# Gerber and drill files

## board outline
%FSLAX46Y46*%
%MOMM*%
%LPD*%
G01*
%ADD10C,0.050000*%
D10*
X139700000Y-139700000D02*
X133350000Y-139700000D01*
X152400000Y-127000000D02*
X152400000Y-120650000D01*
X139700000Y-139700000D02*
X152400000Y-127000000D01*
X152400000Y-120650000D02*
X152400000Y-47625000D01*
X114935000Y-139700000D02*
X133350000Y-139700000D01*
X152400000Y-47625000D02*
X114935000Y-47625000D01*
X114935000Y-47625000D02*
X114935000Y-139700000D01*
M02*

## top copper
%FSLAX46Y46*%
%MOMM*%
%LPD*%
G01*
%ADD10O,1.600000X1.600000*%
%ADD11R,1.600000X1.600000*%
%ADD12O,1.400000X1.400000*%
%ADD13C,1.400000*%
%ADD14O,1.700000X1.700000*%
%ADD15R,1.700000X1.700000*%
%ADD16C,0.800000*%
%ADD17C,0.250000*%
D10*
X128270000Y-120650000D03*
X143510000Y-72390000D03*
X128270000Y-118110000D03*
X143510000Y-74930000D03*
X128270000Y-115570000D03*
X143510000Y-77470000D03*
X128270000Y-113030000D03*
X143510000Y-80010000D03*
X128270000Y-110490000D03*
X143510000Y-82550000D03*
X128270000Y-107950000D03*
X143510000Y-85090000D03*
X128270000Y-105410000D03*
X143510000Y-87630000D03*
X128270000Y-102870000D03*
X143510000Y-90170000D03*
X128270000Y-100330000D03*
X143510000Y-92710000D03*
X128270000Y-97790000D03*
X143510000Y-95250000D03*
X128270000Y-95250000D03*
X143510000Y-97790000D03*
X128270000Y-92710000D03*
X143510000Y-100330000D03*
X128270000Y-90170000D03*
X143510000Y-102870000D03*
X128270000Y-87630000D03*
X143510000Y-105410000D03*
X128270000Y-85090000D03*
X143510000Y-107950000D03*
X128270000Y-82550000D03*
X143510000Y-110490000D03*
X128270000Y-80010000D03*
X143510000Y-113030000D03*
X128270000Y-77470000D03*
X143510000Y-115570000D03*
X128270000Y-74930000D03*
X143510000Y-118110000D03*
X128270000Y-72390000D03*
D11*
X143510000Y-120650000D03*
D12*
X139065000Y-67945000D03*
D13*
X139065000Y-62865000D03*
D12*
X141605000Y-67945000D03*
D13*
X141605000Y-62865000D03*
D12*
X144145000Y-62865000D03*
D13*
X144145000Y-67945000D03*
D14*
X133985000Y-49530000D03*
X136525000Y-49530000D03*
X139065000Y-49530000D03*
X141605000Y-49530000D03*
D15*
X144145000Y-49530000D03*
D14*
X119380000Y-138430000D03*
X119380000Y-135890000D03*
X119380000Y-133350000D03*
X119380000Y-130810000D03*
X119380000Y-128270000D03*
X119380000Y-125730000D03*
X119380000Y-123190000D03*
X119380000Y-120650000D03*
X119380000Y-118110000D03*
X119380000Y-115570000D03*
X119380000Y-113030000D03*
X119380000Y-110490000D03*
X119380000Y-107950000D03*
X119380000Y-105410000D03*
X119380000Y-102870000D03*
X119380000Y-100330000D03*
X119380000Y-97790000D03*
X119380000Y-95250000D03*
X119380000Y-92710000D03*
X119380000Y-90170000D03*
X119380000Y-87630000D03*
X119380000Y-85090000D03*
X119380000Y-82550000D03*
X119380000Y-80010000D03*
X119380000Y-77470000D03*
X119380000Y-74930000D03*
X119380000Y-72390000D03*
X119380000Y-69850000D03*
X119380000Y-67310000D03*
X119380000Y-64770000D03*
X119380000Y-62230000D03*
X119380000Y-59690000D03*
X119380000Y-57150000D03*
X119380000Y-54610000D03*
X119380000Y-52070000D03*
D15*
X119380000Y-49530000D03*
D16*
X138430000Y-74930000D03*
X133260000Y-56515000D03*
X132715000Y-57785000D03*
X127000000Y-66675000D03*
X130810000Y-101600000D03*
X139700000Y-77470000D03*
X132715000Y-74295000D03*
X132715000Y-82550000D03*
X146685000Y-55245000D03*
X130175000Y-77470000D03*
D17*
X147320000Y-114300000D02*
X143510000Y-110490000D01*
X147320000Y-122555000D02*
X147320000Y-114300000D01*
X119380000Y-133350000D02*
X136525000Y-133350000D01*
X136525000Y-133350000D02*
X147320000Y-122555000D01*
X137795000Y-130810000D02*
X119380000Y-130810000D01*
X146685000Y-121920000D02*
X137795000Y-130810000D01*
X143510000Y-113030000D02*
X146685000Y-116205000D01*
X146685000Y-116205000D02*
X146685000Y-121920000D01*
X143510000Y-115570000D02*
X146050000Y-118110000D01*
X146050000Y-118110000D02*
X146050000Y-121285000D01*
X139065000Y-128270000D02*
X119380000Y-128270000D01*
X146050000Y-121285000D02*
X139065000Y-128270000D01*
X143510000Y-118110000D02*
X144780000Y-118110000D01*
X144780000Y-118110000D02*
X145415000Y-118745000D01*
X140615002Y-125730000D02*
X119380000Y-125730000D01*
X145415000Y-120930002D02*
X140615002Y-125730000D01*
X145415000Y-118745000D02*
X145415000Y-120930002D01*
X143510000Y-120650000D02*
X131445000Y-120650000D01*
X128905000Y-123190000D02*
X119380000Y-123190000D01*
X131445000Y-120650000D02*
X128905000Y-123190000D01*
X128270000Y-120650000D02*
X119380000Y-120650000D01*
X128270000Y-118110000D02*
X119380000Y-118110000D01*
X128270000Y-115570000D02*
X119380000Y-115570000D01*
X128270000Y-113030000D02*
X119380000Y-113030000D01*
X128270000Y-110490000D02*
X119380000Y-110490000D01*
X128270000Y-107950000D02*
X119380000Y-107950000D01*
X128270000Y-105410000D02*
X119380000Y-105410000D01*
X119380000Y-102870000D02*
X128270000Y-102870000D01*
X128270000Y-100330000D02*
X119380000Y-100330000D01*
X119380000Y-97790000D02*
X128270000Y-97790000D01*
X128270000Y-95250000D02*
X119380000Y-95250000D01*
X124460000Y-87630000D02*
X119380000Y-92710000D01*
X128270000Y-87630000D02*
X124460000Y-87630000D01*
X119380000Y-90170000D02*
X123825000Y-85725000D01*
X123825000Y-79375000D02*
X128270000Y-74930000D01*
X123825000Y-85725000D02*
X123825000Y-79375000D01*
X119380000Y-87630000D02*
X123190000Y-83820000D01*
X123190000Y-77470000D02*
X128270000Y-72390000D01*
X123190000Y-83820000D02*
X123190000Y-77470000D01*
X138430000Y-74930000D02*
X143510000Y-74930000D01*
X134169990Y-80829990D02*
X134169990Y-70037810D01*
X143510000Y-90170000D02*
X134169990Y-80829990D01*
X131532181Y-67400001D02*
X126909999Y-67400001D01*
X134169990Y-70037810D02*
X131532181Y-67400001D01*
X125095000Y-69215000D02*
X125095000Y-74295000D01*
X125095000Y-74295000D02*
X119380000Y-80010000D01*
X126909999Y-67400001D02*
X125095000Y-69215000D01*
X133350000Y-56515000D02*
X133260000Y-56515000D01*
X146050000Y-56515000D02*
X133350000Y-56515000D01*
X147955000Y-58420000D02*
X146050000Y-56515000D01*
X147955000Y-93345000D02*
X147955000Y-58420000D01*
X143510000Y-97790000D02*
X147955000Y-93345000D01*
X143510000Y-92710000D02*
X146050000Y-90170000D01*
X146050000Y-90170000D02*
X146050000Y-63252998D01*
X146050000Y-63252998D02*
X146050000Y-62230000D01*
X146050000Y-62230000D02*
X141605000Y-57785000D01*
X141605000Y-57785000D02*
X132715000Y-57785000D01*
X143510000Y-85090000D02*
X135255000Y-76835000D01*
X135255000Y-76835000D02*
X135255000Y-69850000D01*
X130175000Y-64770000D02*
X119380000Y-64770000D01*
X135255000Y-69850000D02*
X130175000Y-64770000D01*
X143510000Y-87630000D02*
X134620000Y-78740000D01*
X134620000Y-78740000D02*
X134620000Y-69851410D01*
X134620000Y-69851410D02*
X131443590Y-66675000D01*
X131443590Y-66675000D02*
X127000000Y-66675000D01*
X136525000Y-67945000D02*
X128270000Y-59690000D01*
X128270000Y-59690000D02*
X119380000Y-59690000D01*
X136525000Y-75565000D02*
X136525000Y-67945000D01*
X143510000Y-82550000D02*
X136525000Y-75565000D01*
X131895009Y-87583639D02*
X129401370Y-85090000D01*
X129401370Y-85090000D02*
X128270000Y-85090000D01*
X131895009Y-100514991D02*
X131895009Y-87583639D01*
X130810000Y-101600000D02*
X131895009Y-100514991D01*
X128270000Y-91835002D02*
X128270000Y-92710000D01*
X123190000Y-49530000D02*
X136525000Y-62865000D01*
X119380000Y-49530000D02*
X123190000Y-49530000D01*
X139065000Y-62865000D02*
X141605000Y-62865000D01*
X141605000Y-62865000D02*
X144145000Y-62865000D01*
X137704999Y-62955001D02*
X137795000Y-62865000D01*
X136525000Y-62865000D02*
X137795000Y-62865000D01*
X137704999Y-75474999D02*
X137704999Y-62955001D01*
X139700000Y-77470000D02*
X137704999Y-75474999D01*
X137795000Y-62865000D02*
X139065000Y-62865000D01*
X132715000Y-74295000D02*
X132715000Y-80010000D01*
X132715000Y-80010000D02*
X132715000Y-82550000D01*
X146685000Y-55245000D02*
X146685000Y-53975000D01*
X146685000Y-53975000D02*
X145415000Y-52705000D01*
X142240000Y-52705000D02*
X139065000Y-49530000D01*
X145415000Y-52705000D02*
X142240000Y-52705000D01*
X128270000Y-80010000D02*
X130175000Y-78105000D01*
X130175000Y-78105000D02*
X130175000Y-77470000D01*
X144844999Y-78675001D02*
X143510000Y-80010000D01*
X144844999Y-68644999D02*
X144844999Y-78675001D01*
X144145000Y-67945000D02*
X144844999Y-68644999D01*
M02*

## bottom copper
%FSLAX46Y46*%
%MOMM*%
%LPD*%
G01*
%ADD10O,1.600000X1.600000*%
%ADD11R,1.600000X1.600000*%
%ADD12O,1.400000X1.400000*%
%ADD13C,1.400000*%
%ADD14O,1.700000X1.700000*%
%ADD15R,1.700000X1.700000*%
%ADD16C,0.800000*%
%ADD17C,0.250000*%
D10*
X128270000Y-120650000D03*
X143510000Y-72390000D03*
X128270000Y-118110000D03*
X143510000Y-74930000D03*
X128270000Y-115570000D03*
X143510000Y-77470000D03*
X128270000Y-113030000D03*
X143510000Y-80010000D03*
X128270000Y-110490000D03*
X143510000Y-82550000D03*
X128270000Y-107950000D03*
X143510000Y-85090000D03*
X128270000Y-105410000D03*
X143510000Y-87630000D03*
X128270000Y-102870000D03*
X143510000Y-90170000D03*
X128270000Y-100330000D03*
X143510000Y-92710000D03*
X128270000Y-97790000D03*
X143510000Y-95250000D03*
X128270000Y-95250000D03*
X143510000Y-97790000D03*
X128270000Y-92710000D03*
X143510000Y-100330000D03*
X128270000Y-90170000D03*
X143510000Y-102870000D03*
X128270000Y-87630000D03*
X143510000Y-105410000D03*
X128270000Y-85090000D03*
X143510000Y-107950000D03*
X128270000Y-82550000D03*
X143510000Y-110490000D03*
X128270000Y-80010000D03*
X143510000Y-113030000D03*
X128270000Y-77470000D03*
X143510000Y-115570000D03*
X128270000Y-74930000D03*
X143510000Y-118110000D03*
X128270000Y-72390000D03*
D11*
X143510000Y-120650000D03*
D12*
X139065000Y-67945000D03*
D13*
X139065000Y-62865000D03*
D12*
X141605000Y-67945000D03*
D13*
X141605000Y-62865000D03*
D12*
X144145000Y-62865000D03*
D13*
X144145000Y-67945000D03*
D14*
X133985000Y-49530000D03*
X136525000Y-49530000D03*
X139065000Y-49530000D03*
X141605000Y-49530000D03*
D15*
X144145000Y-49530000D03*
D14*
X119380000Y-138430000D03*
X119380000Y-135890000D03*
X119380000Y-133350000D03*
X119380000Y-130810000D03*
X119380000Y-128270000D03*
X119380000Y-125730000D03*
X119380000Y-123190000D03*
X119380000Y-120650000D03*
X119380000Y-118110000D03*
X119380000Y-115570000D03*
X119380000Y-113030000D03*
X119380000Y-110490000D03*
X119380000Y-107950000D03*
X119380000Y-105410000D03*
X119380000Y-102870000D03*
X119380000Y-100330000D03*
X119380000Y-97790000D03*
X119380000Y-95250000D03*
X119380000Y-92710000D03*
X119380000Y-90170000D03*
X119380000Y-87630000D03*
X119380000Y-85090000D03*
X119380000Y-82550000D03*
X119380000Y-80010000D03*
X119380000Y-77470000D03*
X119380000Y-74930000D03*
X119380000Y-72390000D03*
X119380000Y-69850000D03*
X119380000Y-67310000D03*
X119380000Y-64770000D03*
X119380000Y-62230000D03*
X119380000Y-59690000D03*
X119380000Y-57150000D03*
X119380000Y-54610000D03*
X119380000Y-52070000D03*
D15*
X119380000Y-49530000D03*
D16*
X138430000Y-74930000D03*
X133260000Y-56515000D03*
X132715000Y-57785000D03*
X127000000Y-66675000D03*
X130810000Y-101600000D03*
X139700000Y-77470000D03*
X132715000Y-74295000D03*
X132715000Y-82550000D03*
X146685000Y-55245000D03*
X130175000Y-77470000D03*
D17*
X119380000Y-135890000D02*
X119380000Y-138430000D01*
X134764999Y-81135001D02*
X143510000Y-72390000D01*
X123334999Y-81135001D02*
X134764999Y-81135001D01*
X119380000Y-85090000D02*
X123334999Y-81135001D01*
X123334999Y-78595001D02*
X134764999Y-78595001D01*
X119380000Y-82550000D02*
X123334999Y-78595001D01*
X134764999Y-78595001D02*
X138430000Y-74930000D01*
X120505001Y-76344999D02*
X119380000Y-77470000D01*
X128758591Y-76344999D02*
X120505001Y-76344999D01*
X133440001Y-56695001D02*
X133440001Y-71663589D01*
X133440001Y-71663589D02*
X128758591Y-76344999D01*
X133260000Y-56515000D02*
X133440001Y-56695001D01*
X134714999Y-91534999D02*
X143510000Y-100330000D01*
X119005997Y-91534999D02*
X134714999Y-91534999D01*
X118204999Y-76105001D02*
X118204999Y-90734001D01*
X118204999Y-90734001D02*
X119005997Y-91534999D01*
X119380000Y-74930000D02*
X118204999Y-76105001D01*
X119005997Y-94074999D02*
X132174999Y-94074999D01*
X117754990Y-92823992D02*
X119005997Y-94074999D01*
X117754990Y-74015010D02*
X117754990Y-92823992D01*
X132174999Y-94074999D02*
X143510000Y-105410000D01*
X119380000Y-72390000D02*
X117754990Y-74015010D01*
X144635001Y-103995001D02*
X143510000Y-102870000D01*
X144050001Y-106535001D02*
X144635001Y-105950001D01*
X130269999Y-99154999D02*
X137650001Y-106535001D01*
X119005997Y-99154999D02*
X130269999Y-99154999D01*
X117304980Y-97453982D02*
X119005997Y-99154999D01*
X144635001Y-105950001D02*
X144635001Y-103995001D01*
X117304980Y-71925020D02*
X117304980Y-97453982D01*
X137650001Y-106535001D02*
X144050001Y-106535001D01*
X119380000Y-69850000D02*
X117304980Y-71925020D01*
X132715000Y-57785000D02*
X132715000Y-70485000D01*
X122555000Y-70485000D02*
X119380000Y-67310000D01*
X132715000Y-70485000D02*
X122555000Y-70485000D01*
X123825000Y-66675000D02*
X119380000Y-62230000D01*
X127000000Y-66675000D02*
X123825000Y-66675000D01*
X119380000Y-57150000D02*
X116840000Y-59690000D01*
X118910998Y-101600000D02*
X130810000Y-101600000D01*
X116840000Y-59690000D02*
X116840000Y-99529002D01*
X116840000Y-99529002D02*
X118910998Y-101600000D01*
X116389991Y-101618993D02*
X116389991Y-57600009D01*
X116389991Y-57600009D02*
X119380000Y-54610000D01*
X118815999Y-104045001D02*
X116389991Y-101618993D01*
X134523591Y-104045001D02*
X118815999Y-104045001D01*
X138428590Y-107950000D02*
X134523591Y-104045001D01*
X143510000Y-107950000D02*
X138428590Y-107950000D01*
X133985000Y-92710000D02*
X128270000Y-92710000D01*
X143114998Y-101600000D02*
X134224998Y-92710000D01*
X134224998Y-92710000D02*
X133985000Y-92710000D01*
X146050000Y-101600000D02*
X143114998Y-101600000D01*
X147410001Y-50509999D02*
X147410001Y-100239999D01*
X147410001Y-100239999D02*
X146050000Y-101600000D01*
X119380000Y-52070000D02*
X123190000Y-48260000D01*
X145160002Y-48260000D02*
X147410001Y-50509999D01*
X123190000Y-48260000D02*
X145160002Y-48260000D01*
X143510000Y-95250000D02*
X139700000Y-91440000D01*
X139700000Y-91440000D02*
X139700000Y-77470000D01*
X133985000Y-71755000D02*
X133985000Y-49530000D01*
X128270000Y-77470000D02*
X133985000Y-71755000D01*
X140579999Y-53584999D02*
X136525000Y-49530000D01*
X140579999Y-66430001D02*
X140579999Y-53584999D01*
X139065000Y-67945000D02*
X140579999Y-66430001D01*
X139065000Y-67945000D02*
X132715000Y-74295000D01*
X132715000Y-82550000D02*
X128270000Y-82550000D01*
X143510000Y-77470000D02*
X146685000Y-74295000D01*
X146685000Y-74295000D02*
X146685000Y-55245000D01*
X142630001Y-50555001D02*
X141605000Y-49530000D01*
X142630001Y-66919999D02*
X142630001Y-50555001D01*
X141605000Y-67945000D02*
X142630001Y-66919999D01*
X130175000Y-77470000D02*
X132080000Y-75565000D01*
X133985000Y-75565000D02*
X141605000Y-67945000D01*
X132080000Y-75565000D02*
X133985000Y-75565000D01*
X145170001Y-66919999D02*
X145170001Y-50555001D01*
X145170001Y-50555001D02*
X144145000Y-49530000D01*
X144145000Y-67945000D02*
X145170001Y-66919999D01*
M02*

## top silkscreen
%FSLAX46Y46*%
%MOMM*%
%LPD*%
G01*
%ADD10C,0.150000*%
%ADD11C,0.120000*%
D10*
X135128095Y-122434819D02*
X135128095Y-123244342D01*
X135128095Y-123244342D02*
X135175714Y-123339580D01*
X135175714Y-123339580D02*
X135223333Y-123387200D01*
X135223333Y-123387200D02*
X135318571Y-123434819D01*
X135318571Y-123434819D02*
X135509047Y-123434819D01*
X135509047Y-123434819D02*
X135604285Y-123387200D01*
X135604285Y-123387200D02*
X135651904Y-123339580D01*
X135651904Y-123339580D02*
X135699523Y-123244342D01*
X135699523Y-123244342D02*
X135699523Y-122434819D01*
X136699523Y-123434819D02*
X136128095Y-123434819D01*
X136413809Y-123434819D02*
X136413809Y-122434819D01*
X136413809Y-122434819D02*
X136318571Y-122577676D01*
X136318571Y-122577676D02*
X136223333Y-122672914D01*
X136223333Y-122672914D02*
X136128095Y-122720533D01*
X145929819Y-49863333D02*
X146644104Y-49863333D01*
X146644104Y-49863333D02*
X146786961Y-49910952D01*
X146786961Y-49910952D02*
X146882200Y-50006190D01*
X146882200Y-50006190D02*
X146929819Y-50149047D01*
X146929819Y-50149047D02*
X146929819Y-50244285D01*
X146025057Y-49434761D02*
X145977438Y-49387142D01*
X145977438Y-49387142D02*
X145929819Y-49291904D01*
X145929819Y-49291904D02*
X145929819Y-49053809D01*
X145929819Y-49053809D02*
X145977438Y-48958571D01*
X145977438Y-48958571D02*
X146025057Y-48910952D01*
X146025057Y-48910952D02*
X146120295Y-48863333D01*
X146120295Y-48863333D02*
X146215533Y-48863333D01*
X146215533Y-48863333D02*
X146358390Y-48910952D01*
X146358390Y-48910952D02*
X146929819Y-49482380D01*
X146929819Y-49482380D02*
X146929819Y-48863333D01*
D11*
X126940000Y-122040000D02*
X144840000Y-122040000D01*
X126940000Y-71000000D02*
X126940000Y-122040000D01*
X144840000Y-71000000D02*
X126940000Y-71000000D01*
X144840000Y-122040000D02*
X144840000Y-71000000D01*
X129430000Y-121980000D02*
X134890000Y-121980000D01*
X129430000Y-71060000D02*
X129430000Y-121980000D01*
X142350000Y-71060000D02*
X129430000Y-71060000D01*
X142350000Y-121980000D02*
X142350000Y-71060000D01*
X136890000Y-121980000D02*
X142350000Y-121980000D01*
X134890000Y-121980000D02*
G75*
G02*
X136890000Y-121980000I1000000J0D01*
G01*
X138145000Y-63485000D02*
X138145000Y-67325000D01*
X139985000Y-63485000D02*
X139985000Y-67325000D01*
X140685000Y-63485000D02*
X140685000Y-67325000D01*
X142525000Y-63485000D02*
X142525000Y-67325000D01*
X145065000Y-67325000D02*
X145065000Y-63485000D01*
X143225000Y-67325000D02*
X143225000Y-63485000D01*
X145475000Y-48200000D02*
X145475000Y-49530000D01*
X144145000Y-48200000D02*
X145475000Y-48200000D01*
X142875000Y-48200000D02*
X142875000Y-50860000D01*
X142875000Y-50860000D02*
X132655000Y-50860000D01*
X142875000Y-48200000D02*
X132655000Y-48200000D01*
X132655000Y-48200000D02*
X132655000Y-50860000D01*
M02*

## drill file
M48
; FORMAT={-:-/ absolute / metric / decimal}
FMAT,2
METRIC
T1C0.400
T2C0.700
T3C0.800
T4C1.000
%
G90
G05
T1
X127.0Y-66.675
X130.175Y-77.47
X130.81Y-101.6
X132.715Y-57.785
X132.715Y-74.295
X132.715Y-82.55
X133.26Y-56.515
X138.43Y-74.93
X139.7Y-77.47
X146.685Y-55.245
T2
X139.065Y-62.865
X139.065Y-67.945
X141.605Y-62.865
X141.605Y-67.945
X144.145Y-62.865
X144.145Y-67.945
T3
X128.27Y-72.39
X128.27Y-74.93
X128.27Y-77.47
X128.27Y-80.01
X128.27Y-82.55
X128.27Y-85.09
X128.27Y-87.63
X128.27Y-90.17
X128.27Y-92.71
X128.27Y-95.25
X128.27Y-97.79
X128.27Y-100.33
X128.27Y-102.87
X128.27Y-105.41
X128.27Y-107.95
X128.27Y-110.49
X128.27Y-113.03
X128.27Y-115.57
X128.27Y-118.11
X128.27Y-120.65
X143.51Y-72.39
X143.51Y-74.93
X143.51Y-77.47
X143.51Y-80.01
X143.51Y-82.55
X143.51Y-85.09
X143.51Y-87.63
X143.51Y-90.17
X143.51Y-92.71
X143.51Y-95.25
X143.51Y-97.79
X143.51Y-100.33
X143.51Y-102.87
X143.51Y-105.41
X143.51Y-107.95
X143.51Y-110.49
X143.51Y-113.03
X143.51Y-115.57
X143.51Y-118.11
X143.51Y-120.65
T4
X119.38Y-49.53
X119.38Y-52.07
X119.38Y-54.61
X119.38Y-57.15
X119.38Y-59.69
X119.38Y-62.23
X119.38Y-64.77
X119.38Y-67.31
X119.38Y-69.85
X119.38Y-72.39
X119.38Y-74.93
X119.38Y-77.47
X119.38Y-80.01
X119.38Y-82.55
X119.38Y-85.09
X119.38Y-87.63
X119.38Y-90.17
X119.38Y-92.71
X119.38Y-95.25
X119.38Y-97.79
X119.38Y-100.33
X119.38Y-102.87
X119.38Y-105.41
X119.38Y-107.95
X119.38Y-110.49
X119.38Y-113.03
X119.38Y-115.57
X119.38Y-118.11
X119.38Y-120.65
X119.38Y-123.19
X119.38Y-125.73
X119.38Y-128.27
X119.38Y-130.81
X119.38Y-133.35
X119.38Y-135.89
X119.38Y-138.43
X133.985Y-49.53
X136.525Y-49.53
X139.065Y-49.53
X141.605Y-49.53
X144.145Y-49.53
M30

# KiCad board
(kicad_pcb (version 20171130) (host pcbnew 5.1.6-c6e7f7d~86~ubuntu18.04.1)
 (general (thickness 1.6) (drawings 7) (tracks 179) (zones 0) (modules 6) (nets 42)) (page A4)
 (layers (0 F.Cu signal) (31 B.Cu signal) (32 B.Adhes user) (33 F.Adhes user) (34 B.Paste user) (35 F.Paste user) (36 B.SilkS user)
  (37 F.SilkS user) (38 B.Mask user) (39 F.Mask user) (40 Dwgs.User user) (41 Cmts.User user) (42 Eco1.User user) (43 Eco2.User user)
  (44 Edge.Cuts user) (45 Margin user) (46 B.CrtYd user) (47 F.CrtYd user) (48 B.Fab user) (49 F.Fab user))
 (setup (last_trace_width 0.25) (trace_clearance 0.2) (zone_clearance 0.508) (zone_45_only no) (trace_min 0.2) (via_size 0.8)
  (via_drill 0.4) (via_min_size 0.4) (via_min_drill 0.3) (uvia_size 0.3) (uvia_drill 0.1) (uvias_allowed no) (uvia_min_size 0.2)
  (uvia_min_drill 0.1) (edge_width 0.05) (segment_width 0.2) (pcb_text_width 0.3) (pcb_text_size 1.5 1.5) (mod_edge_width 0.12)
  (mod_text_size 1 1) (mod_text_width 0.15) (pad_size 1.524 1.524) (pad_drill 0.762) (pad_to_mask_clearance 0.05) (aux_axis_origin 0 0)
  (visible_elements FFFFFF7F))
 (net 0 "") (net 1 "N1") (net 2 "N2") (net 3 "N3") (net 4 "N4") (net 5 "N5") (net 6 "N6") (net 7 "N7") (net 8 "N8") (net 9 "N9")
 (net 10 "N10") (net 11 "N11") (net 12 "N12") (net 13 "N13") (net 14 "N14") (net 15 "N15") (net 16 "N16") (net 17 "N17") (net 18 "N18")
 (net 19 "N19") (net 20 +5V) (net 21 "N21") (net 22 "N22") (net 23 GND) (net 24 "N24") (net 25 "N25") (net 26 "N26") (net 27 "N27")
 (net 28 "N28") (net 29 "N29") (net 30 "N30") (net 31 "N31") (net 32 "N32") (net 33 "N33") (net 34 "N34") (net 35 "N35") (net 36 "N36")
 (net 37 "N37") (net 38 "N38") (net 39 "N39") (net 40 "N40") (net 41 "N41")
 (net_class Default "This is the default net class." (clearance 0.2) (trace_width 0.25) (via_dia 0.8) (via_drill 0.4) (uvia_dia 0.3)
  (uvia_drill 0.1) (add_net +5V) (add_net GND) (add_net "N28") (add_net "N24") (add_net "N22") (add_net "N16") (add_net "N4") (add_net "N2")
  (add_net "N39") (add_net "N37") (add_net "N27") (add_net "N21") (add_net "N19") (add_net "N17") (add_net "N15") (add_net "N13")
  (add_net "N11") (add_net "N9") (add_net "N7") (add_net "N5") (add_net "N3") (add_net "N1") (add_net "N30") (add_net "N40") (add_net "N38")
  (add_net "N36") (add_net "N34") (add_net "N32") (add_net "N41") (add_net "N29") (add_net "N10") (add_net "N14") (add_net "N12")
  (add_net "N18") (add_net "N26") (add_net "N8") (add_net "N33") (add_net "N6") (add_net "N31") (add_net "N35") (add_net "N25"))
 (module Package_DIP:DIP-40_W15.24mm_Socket (layer F.Cu) (at 143.51 120.65 180)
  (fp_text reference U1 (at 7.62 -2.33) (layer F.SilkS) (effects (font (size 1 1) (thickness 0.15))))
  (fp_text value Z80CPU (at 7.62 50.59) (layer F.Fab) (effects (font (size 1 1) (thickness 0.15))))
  (fp_line (start 16.57 -1.39) (end -1.33 -1.39) (layer F.SilkS) (width 0.12))
  (fp_line (start 16.57 49.65) (end 16.57 -1.39) (layer F.SilkS) (width 0.12))
  (fp_line (start -1.33 49.65) (end 16.57 49.65) (layer F.SilkS) (width 0.12))
  (fp_line (start -1.33 -1.39) (end -1.33 49.65) (layer F.SilkS) (width 0.12))
  (fp_line (start 14.08 -1.33) (end 8.62 -1.33) (layer F.SilkS) (width 0.12))
  (fp_line (start 14.08 49.59) (end 14.08 -1.33) (layer F.SilkS) (width 0.12))
  (fp_line (start 1.16 49.59) (end 14.08 49.59) (layer F.SilkS) (width 0.12))
  (fp_line (start 1.16 -1.33) (end 1.16 49.59) (layer F.SilkS) (width 0.12))
  (fp_line (start 6.62 -1.33) (end 1.16 -1.33) (layer F.SilkS) (width 0.12))
  (fp_arc (start 7.62 -1.33) (end 6.62 -1.33) (angle -180) (layer F.SilkS) (width 0.12))
  (pad 40 thru_hole oval (at 15.24 0 180) (size 1.6 1.6) (drill 0.8) (layers *.Cu *.Mask) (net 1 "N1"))
  (pad 20 thru_hole oval (at 0 48.26 180) (size 1.6 1.6) (drill 0.8) (layers *.Cu *.Mask) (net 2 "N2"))
  (pad 39 thru_hole oval (at 15.24 2.54 180) (size 1.6 1.6) (drill 0.8) (layers *.Cu *.Mask) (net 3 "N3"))
  (pad 19 thru_hole oval (at 0 45.72 180) (size 1.6 1.6) (drill 0.8) (layers *.Cu *.Mask) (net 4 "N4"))
  (pad 38 thru_hole oval (at 15.24 5.08 180) (size 1.6 1.6) (drill 0.8) (layers *.Cu *.Mask) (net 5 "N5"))
  (pad 18 thru_hole oval (at 0 43.18 180) (size 1.6 1.6) (drill 0.8) (layers *.Cu *.Mask) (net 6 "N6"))
  (pad 37 thru_hole oval (at 15.24 7.62 180) (size 1.6 1.6) (drill 0.8) (layers *.Cu *.Mask) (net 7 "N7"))
  (pad 17 thru_hole oval (at 0 40.64 180) (size 1.6 1.6) (drill 0.8) (layers *.Cu *.Mask) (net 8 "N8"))
  (pad 36 thru_hole oval (at 15.24 10.16 180) (size 1.6 1.6) (drill 0.8) (layers *.Cu *.Mask) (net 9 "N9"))
  (pad 16 thru_hole oval (at 0 38.1 180) (size 1.6 1.6) (drill 0.8) (layers *.Cu *.Mask) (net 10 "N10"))
  (pad 35 thru_hole oval (at 15.24 12.7 180) (size 1.6 1.6) (drill 0.8) (layers *.Cu *.Mask) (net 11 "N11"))
  (pad 15 thru_hole oval (at 0 35.56 180) (size 1.6 1.6) (drill 0.8) (layers *.Cu *.Mask) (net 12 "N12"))
  (pad 34 thru_hole oval (at 15.24 15.24 180) (size 1.6 1.6) (drill 0.8) (layers *.Cu *.Mask) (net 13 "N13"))
  (pad 14 thru_hole oval (at 0 33.02 180) (size 1.6 1.6) (drill 0.8) (layers *.Cu *.Mask) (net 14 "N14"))
  (pad 33 thru_hole oval (at 15.24 17.78 180) (size 1.6 1.6) (drill 0.8) (layers *.Cu *.Mask) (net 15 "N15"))
  (pad 13 thru_hole oval (at 0 30.48 180) (size 1.6 1.6) (drill 0.8) (layers *.Cu *.Mask) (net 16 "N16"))
  (pad 32 thru_hole oval (at 15.24 20.32 180) (size 1.6 1.6) (drill 0.8) (layers *.Cu *.Mask) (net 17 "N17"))
  (pad 12 thru_hole oval (at 0 27.94 180) (size 1.6 1.6) (drill 0.8) (layers *.Cu *.Mask) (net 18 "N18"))
  (pad 31 thru_hole oval (at 15.24 22.86 180) (size 1.6 1.6) (drill 0.8) (layers *.Cu *.Mask) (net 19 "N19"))
  (pad 11 thru_hole oval (at 0 25.4 180) (size 1.6 1.6) (drill 0.8) (layers *.Cu *.Mask) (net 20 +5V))
  (pad 30 thru_hole oval (at 15.24 25.4 180) (size 1.6 1.6) (drill 0.8) (layers *.Cu *.Mask) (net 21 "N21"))
  (pad 10 thru_hole oval (at 0 22.86 180) (size 1.6 1.6) (drill 0.8) (layers *.Cu *.Mask) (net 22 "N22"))
  (pad 29 thru_hole oval (at 15.24 27.94 180) (size 1.6 1.6) (drill 0.8) (layers *.Cu *.Mask) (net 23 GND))
  (pad 9 thru_hole oval (at 0 20.32 180) (size 1.6 1.6) (drill 0.8) (layers *.Cu *.Mask) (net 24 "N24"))
  (pad 28 thru_hole oval (at 15.24 30.48 180) (size 1.6 1.6) (drill 0.8) (layers *.Cu *.Mask) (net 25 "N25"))
  (pad 8 thru_hole oval (at 0 17.78 180) (size 1.6 1.6) (drill 0.8) (layers *.Cu *.Mask) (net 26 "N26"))
  (pad 27 thru_hole oval (at 15.24 33.02 180) (size 1.6 1.6) (drill 0.8) (layers *.Cu *.Mask) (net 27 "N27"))
  (pad 7 thru_hole oval (at 0 15.24 180) (size 1.6 1.6) (drill 0.8) (layers *.Cu *.Mask) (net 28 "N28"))
  (pad 26 thru_hole oval (at 15.24 35.56 180) (size 1.6 1.6) (drill 0.8) (layers *.Cu *.Mask) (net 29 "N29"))
  (pad 6 thru_hole oval (at 0 12.7 180) (size 1.6 1.6) (drill 0.8) (layers *.Cu *.Mask) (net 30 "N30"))
  (pad 25 thru_hole oval (at 15.24 38.1 180) (size 1.6 1.6) (drill 0.8) (layers *.Cu *.Mask) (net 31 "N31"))
  (pad 5 thru_hole oval (at 0 10.16 180) (size 1.6 1.6) (drill 0.8) (layers *.Cu *.Mask) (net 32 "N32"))
  (pad 24 thru_hole oval (at 15.24 40.64 180) (size 1.6 1.6) (drill 0.8) (layers *.Cu *.Mask) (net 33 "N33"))
  (pad 4 thru_hole oval (at 0 7.62 180) (size 1.6 1.6) (drill 0.8) (layers *.Cu *.Mask) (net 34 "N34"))
  (pad 23 thru_hole oval (at 15.24 43.18 180) (size 1.6 1.6) (drill 0.8) (layers *.Cu *.Mask) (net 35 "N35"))
  (pad 3 thru_hole oval (at 0 5.08 180) (size 1.6 1.6) (drill 0.8) (layers *.Cu *.Mask) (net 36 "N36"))
  (pad 22 thru_hole oval (at 15.24 45.72 180) (size 1.6 1.6) (drill 0.8) (layers *.Cu *.Mask) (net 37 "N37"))
  (pad 2 thru_hole oval (at 0 2.54 180) (size 1.6 1.6) (drill 0.8) (layers *.Cu *.Mask) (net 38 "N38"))
  (pad 21 thru_hole oval (at 15.24 48.26 180) (size 1.6 1.6) (drill 0.8) (layers *.Cu *.Mask) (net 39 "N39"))
  (pad 1 thru_hole rect (at 0 0 180) (size 1.6 1.6) (drill 0.8) (layers *.Cu *.Mask) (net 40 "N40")))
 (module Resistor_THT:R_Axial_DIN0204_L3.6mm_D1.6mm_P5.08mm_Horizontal (layer F.Cu) (at 139.065 62.865 270)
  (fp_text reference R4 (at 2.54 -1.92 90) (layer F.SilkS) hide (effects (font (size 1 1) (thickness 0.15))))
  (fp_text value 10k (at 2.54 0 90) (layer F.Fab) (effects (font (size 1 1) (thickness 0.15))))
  (fp_line (start 0.62 0.92) (end 4.46 0.92) (layer F.SilkS) (width 0.12))
  (fp_line (start 0.62 -0.92) (end 4.46 -0.92) (layer F.SilkS) (width 0.12))
  (pad 2 thru_hole oval (at 5.08 0 270) (size 1.4 1.4) (drill 0.7) (layers *.Cu *.Mask) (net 31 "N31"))
  (pad 1 thru_hole circle (at 0 0 270) (size 1.4 1.4) (drill 0.7) (layers *.Cu *.Mask) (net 20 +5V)))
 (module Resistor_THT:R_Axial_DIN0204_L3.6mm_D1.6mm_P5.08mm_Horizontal (layer F.Cu) (at 141.605 62.865 270)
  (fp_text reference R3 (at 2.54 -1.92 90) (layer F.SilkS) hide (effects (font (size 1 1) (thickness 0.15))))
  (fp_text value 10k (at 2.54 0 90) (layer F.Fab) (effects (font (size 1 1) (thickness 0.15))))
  (fp_line (start 0.62 0.92) (end 4.46 0.92) (layer F.SilkS) (width 0.12))
  (fp_line (start 0.62 -0.92) (end 4.46 -0.92) (layer F.SilkS) (width 0.12))
  (pad 2 thru_hole oval (at 5.08 0 270) (size 1.4 1.4) (drill 0.7) (layers *.Cu *.Mask) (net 33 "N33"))
  (pad 1 thru_hole circle (at 0 0 270) (size 1.4 1.4) (drill 0.7) (layers *.Cu *.Mask) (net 20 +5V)))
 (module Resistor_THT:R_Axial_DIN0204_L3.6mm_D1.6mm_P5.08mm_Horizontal (layer F.Cu) (at 144.145 67.945 90)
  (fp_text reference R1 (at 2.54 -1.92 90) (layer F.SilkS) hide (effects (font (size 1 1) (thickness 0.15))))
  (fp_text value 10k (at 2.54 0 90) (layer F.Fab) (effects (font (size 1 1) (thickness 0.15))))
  (fp_line (start 0.62 0.92) (end 4.46 0.92) (layer F.SilkS) (width 0.12))
  (fp_line (start 0.62 -0.92) (end 4.46 -0.92) (layer F.SilkS) (width 0.12))
  (pad 2 thru_hole oval (at 5.08 0 90) (size 1.4 1.4) (drill 0.7) (layers *.Cu *.Mask) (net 20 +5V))
  (pad 1 thru_hole circle (at 0 0 90) (size 1.4 1.4) (drill 0.7) (layers *.Cu *.Mask) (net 8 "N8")))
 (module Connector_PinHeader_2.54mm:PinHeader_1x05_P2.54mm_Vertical (layer F.Cu) (at 144.145 49.53 270)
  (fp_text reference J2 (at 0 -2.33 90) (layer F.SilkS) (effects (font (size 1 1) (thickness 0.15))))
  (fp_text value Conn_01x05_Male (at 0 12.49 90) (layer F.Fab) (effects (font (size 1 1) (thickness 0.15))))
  (fp_line (start -1.33 -1.33) (end 0 -1.33) (layer F.SilkS) (width 0.12))
  (fp_line (start -1.33 0) (end -1.33 -1.33) (layer F.SilkS) (width 0.12))
  (fp_line (start -1.33 1.27) (end 1.33 1.27) (layer F.SilkS) (width 0.12))
  (fp_line (start 1.33 1.27) (end 1.33 11.49) (layer F.SilkS) (width 0.12))
  (fp_line (start -1.33 1.27) (end -1.33 11.49) (layer F.SilkS) (width 0.12))
  (fp_line (start -1.33 11.49) (end 1.33 11.49) (layer F.SilkS) (width 0.12))
  (pad 5 thru_hole oval (at 0 10.16 270) (size 1.7 1.7) (drill 1) (layers *.Cu *.Mask) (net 35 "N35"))
  (pad 4 thru_hole oval (at 0 7.62 270) (size 1.7 1.7) (drill 1) (layers *.Cu *.Mask) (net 31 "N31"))
  (pad 3 thru_hole oval (at 0 5.08 270) (size 1.7 1.7) (drill 1) (layers *.Cu *.Mask) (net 6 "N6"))
  (pad 2 thru_hole oval (at 0 2.54 270) (size 1.7 1.7) (drill 1) (layers *.Cu *.Mask) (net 33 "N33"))
  (pad 1 thru_hole rect (at 0 0 270) (size 1.7 1.7) (drill 1) (layers *.Cu *.Mask) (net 8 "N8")))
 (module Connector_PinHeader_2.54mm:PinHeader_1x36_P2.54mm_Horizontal (layer B.Cu) (at 119.38 49.53 180)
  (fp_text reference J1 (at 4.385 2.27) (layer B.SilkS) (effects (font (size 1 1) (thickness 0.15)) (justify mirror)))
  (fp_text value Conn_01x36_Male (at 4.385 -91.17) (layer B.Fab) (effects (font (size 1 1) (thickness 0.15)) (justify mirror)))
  (pad 36 thru_hole oval (at 0 -88.9 180) (size 1.7 1.7) (drill 1) (layers *.Cu *.Mask) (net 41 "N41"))
  (pad 35 thru_hole oval (at 0 -86.36 180) (size 1.7 1.7) (drill 1) (layers *.Cu *.Mask) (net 41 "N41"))
  (pad 34 thru_hole oval (at 0 -83.82 180) (size 1.7 1.7) (drill 1) (layers *.Cu *.Mask) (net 32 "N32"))
  (pad 33 thru_hole oval (at 0 -81.28 180) (size 1.7 1.7) (drill 1) (layers *.Cu *.Mask) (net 34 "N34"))
  (pad 32 thru_hole oval (at 0 -78.74 180) (size 1.7 1.7) (drill 1) (layers *.Cu *.Mask) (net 36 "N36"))
  (pad 31 thru_hole oval (at 0 -76.2 180) (size 1.7 1.7) (drill 1) (layers *.Cu *.Mask) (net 38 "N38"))
  (pad 30 thru_hole oval (at 0 -73.66 180) (size 1.7 1.7) (drill 1) (layers *.Cu *.Mask) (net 40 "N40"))
  (pad 29 thru_hole oval (at 0 -71.12 180) (size 1.7 1.7) (drill 1) (layers *.Cu *.Mask) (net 1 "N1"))
  (pad 28 thru_hole oval (at 0 -68.58 180) (size 1.7 1.7) (drill 1) (layers *.Cu *.Mask) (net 3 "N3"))
  (pad 27 thru_hole oval (at 0 -66.04 180) (size 1.7 1.7) (drill 1) (layers *.Cu *.Mask) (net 5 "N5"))
  (pad 26 thru_hole oval (at 0 -63.5 180) (size 1.7 1.7) (drill 1) (layers *.Cu *.Mask) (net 7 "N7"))
  (pad 25 thru_hole oval (at 0 -60.96 180) (size 1.7 1.7) (drill 1) (layers *.Cu *.Mask) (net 9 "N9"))
  (pad 24 thru_hole oval (at 0 -58.42 180) (size 1.7 1.7) (drill 1) (layers *.Cu *.Mask) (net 11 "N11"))
  (pad 23 thru_hole oval (at 0 -55.88 180) (size 1.7 1.7) (drill 1) (layers *.Cu *.Mask) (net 13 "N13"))
  (pad 22 thru_hole oval (at 0 -53.34 180) (size 1.7 1.7) (drill 1) (layers *.Cu *.Mask) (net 15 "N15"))
  (pad 21 thru_hole oval (at 0 -50.8 180) (size 1.7 1.7) (drill 1) (layers *.Cu *.Mask) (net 17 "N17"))
  (pad 20 thru_hole oval (at 0 -48.26 180) (size 1.7 1.7) (drill 1) (layers *.Cu *.Mask) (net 19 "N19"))
  (pad 19 thru_hole oval (at 0 -45.72 180) (size 1.7 1.7) (drill 1) (layers *.Cu *.Mask) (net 21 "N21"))
  (pad 18 thru_hole oval (at 0 -43.18 180) (size 1.7 1.7) (drill 1) (layers *.Cu *.Mask) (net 27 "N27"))
  (pad 17 thru_hole oval (at 0 -40.64 180) (size 1.7 1.7) (drill 1) (layers *.Cu *.Mask) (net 37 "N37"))
  (pad 16 thru_hole oval (at 0 -38.1 180) (size 1.7 1.7) (drill 1) (layers *.Cu *.Mask) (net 39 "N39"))
  (pad 15 thru_hole oval (at 0 -35.56 180) (size 1.7 1.7) (drill 1) (layers *.Cu *.Mask) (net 2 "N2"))
  (pad 14 thru_hole oval (at 0 -33.02 180) (size 1.7 1.7) (drill 1) (layers *.Cu *.Mask) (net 4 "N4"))
  (pad 13 thru_hole oval (at 0 -30.48 180) (size 1.7 1.7) (drill 1) (layers *.Cu *.Mask) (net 16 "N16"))
  (pad 12 thru_hole oval (at 0 -27.94 180) (size 1.7 1.7) (drill 1) (layers *.Cu *.Mask) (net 22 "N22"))
  (pad 11 thru_hole oval (at 0 -25.4 180) (size 1.7 1.7) (drill 1) (layers *.Cu *.Mask) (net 24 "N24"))
  (pad 10 thru_hole oval (at 0 -22.86 180) (size 1.7 1.7) (drill 1) (layers *.Cu *.Mask) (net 28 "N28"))
  (pad 9 thru_hole oval (at 0 -20.32 180) (size 1.7 1.7) (drill 1) (layers *.Cu *.Mask) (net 26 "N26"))
  (pad 8 thru_hole oval (at 0 -17.78 180) (size 1.7 1.7) (drill 1) (layers *.Cu *.Mask) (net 18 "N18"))
  (pad 7 thru_hole oval (at 0 -15.24 180) (size 1.7 1.7) (drill 1) (layers *.Cu *.Mask) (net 12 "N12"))
  (pad 6 thru_hole oval (at 0 -12.7 180) (size 1.7 1.7) (drill 1) (layers *.Cu *.Mask) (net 14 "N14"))
  (pad 5 thru_hole oval (at 0 -10.16 180) (size 1.7 1.7) (drill 1) (layers *.Cu *.Mask) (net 10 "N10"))
  (pad 4 thru_hole oval (at 0 -7.62 180) (size 1.7 1.7) (drill 1) (layers *.Cu *.Mask) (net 29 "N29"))
  (pad 3 thru_hole oval (at 0 -5.08 180) (size 1.7 1.7) (drill 1) (layers *.Cu *.Mask) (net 30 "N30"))
  (pad 2 thru_hole oval (at 0 -2.54 180) (size 1.7 1.7) (drill 1) (layers *.Cu *.Mask) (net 23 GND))
  (pad 1 thru_hole rect (at 0 0 180) (size 1.7 1.7) (drill 1) (layers *.Cu *.Mask) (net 20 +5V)))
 (gr_line (start 139.7 139.7) (end 133.35 139.7) (layer Edge.Cuts) (width 0.05))
 (gr_line (start 152.4 127) (end 152.4 120.65) (layer Edge.Cuts) (width 0.05))
 (gr_line (start 139.7 139.7) (end 152.4 127) (layer Edge.Cuts) (width 0.05))
 (gr_line (start 152.4 120.65) (end 152.4 47.625) (layer Edge.Cuts) (width 0.05))
 (gr_line (start 114.935 139.7) (end 133.35 139.7) (layer Edge.Cuts) (width 0.05))
 (gr_line (start 152.4 47.625) (end 114.935 47.625) (layer Edge.Cuts) (width 0.05))
 (gr_line (start 114.935 47.625) (end 114.935 139.7) (layer Edge.Cuts) (width 0.05))
 (segment (start 119.38 135.89) (end 119.38 138.43) (width 0.25) (layer B.Cu) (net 41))
 (segment (start 147.32 114.3) (end 143.51 110.49) (width 0.25) (layer F.Cu) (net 32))
 (segment (start 147.32 122.555) (end 147.32 114.3) (width 0.25) (layer F.Cu) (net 32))
 (segment (start 119.38 133.35) (end 136.525 133.35) (width 0.25) (layer F.Cu) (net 32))
 (segment (start 136.525 133.35) (end 147.32 122.555) (width 0.25) (layer F.Cu) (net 32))
 (segment (start 137.795 130.81) (end 119.38 130.81) (width 0.25) (layer F.Cu) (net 34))
 (segment (start 146.685 121.92) (end 137.795 130.81) (width 0.25) (layer F.Cu) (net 34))
 (segment (start 143.51 113.03) (end 146.685 116.205) (width 0.25) (layer F.Cu) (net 34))
 (segment (start 146.685 116.205) (end 146.685 121.92) (width 0.25) (layer F.Cu) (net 34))
 (segment (start 143.51 115.57) (end 146.05 118.11) (width 0.25) (layer F.Cu) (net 36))
 (segment (start 146.05 118.11) (end 146.05 121.285) (width 0.25) (layer F.Cu) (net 36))
 (segment (start 139.065 128.27) (end 119.38 128.27) (width 0.25) (layer F.Cu) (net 36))
 (segment (start 146.05 121.285) (end 139.065 128.27) (width 0.25) (layer F.Cu) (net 36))
 (segment (start 143.51 118.11) (end 144.78 118.11) (width 0.25) (layer F.Cu) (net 38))
 (segment (start 144.78 118.11) (end 145.415 118.745) (width 0.25) (layer F.Cu) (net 38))
 (segment (start 140.615002 125.73) (end 119.38 125.73) (width 0.25) (layer F.Cu) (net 38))
 (segment (start 145.415 120.930002) (end 140.615002 125.73) (width 0.25) (layer F.Cu) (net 38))
 (segment (start 145.415 118.745) (end 145.415 120.930002) (width 0.25) (layer F.Cu) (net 38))
 (segment (start 143.51 120.65) (end 131.445 120.65) (width 0.25) (layer F.Cu) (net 40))
 (segment (start 128.905 123.19) (end 119.38 123.19) (width 0.25) (layer F.Cu) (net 40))
 (segment (start 131.445 120.65) (end 128.905 123.19) (width 0.25) (layer F.Cu) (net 40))
 (segment (start 128.27 120.65) (end 119.38 120.65) (width 0.25) (layer F.Cu) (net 1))
 (segment (start 128.27 118.11) (end 119.38 118.11) (width 0.25) (layer F.Cu) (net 3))
 (segment (start 128.27 115.57) (end 119.38 115.57) (width 0.25) (layer F.Cu) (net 5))
 (segment (start 128.27 113.03) (end 119.38 113.03) (width 0.25) (layer F.Cu) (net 7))
 (segment (start 128.27 110.49) (end 119.38 110.49) (width 0.25) (layer F.Cu) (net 9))
 (segment (start 128.27 107.95) (end 119.38 107.95) (width 0.25) (layer F.Cu) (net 11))
 (segment (start 128.27 105.41) (end 119.38 105.41) (width 0.25) (layer F.Cu) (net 13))
 (segment (start 119.38 102.87) (end 128.27 102.87) (width 0.25) (layer F.Cu) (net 15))
 (segment (start 128.27 100.33) (end 119.38 100.33) (width 0.25) (layer F.Cu) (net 17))
 (segment (start 119.38 97.79) (end 128.27 97.79) (width 0.25) (layer F.Cu) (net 19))
 (segment (start 128.27 95.25) (end 119.38 95.25) (width 0.25) (layer F.Cu) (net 21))
 (segment (start 124.46 87.63) (end 119.38 92.71) (width 0.25) (layer F.Cu) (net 27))
 (segment (start 128.27 87.63) (end 124.46 87.63) (width 0.25) (layer F.Cu) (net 27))
 (segment (start 119.38 90.17) (end 123.825 85.725) (width 0.25) (layer F.Cu) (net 37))
 (segment (start 123.825 79.375) (end 128.27 74.93) (width 0.25) (layer F.Cu) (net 37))
 (segment (start 123.825 85.725) (end 123.825 79.375) (width 0.25) (layer F.Cu) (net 37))
 (segment (start 119.38 87.63) (end 123.19 83.82) (width 0.25) (layer F.Cu) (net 39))
 (segment (start 123.19 77.47) (end 128.27 72.39) (width 0.25) (layer F.Cu) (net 39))
 (segment (start 123.19 83.82) (end 123.19 77.47) (width 0.25) (layer F.Cu) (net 39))
 (segment (start 134.764999 81.135001) (end 143.51 72.39) (width 0.25) (layer B.Cu) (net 2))
 (segment (start 123.334999 81.135001) (end 134.764999 81.135001) (width 0.25) (layer B.Cu) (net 2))
 (segment (start 119.38 85.09) (end 123.334999 81.135001) (width 0.25) (layer B.Cu) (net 2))
 (segment (start 123.334999 78.595001) (end 134.764999 78.595001) (width 0.25) (layer B.Cu) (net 4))
 (segment (start 119.38 82.55) (end 123.334999 78.595001) (width 0.25) (layer B.Cu) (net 4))
 (segment (start 134.764999 78.595001) (end 138.43 74.93) (width 0.25) (layer B.Cu) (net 4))
 (via (at 138.43 74.93) (size 0.8) (drill 0.4) (layers F.Cu B.Cu) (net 4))
 (segment (start 138.43 74.93) (end 143.51 74.93) (width 0.25) (layer F.Cu) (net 4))
 (segment (start 134.16999 80.82999) (end 134.16999 70.03781) (width 0.25) (layer F.Cu) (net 16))
 (segment (start 143.51 90.17) (end 134.16999 80.82999) (width 0.25) (layer F.Cu) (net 16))
 (segment (start 131.532181 67.400001) (end 126.909999 67.400001) (width 0.25) (layer F.Cu) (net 16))
 (segment (start 134.16999 70.03781) (end 131.532181 67.400001) (width 0.25) (layer F.Cu) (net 16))
 (segment (start 125.095 69.215) (end 125.095 74.295) (width 0.25) (layer F.Cu) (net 16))
 (segment (start 125.095 74.295) (end 119.38 80.01) (width 0.25) (layer F.Cu) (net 16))
 (segment (start 126.909999 67.400001) (end 125.095 69.215) (width 0.25) (layer F.Cu) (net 16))
 (segment (start 133.35 56.515) (end 133.26 56.515) (width 0.25) (layer F.Cu) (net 22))
 (segment (start 146.05 56.515) (end 133.35 56.515) (width 0.25) (layer F.Cu) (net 22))
 (segment (start 147.955 58.42) (end 146.05 56.515) (width 0.25) (layer F.Cu) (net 22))
 (via (at 133.26 56.515) (size 0.8) (drill 0.4) (layers F.Cu B.Cu) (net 22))
 (segment (start 147.955 93.345) (end 147.955 58.42) (width 0.25) (layer F.Cu) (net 22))
 (segment (start 143.51 97.79) (end 147.955 93.345) (width 0.25) (layer F.Cu) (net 22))
 (segment (start 120.505001 76.344999) (end 119.38 77.47) (width 0.25) (layer B.Cu) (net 22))
 (segment (start 128.758591 76.344999) (end 120.505001 76.344999) (width 0.25) (layer B.Cu) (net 22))
 (segment (start 133.440001 56.695001) (end 133.440001 71.663589) (width 0.25) (layer B.Cu) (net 22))
 (segment (start 133.440001 71.663589) (end 128.758591 76.344999) (width 0.25) (layer B.Cu) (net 22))
 (segment (start 133.26 56.515) (end 133.440001 56.695001) (width 0.25) (layer B.Cu) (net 22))
 (segment (start 134.714999 91.534999) (end 143.51 100.33) (width 0.25) (layer B.Cu) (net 24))
 (segment (start 119.005997 91.534999) (end 134.714999 91.534999) (width 0.25) (layer B.Cu) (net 24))
 (segment (start 118.204999 76.105001) (end 118.204999 90.734001) (width 0.25) (layer B.Cu) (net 24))
 (segment (start 118.204999 90.734001) (end 119.005997 91.534999) (width 0.25) (layer B.Cu) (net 24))
 (segment (start 119.38 74.93) (end 118.204999 76.105001) (width 0.25) (layer B.Cu) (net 24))
 (segment (start 119.005997 94.074999) (end 132.174999 94.074999) (width 0.25) (layer B.Cu) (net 28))
 (segment (start 117.75499 92.823992) (end 119.005997 94.074999) (width 0.25) (layer B.Cu) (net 28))
 (segment (start 117.75499 74.01501) (end 117.75499 92.823992) (width 0.25) (layer B.Cu) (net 28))
 (segment (start 132.174999 94.074999) (end 143.51 105.41) (width 0.25) (layer B.Cu) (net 28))
 (segment (start 119.38 72.39) (end 117.75499 74.01501) (width 0.25) (layer B.Cu) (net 28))
 (segment (start 144.635001 103.995001) (end 143.51 102.87) (width 0.25) (layer B.Cu) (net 26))
 (segment (start 144.050001 106.535001) (end 144.635001 105.950001) (width 0.25) (layer B.Cu) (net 26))
 (segment (start 130.269999 99.154999) (end 137.650001 106.535001) (width 0.25) (layer B.Cu) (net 26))
 (segment (start 119.005997 99.154999) (end 130.269999 99.154999) (width 0.25) (layer B.Cu) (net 26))
 (segment (start 117.30498 97.453982) (end 119.005997 99.154999) (width 0.25) (layer B.Cu) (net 26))
 (segment (start 144.635001 105.950001) (end 144.635001 103.995001) (width 0.25) (layer B.Cu) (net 26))
 (segment (start 117.30498 71.92502) (end 117.30498 97.453982) (width 0.25) (layer B.Cu) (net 26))
 (segment (start 137.650001 106.535001) (end 144.050001 106.535001) (width 0.25) (layer B.Cu) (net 26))
 (segment (start 119.38 69.85) (end 117.30498 71.92502) (width 0.25) (layer B.Cu) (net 26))
 (segment (start 143.51 92.71) (end 146.05 90.17) (width 0.25) (layer F.Cu) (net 18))
 (segment (start 146.05 90.17) (end 146.05 63.252998) (width 0.25) (layer F.Cu) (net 18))
 (segment (start 146.05 63.252998) (end 146.05 62.23) (width 0.25) (layer F.Cu) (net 18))
 (segment (start 146.05 62.23) (end 141.605 57.785) (width 0.25) (layer F.Cu) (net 18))
 (via (at 132.715 57.785) (size 0.8) (drill 0.4) (layers F.Cu B.Cu) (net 18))
 (segment (start 141.605 57.785) (end 132.715 57.785) (width 0.25) (layer F.Cu) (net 18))
 (segment (start 132.715 57.785) (end 132.715 70.485) (width 0.25) (layer B.Cu) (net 18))
 (segment (start 122.555 70.485) (end 119.38 67.31) (width 0.25) (layer B.Cu) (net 18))
 (segment (start 132.715 70.485) (end 122.555 70.485) (width 0.25) (layer B.Cu) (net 18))
 (segment (start 143.51 85.09) (end 135.255 76.835) (width 0.25) (layer F.Cu) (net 12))
 (segment (start 135.255 76.835) (end 135.255 69.85) (width 0.25) (layer F.Cu) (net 12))
 (segment (start 130.175 64.77) (end 119.38 64.77) (width 0.25) (layer F.Cu) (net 12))
 (segment (start 135.255 69.85) (end 130.175 64.77) (width 0.25) (layer F.Cu) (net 12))
 (segment (start 143.51 87.63) (end 134.62 78.74) (width 0.25) (layer F.Cu) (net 14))
 (segment (start 134.62 78.74) (end 134.62 69.85141) (width 0.25) (layer F.Cu) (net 14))
 (segment (start 134.62 69.85141) (end 131.44359 66.675) (width 0.25) (layer F.Cu) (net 14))
 (via (at 127 66.675) (size 0.8) (drill 0.4) (layers F.Cu B.Cu) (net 14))
 (segment (start 131.44359 66.675) (end 127 66.675) (width 0.25) (layer F.Cu) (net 14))
 (segment (start 123.825 66.675) (end 119.38 62.23) (width 0.25) (layer B.Cu) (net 14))
 (segment (start 127 66.675) (end 123.825 66.675) (width 0.25) (layer B.Cu) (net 14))
 (segment (start 136.525 67.945) (end 128.27 59.69) (width 0.25) (layer F.Cu) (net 10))
 (segment (start 128.27 59.69) (end 119.38 59.69) (width 0.25) (layer F.Cu) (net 10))
 (segment (start 136.525 75.565) (end 136.525 67.945) (width 0.25) (layer F.Cu) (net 10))
 (segment (start 143.51 82.55) (end 136.525 75.565) (width 0.25) (layer F.Cu) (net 10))
 (segment (start 119.38 57.15) (end 116.84 59.69) (width 0.25) (layer B.Cu) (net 29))
 (via (at 130.81 101.6) (size 0.8) (drill 0.4) (layers F.Cu B.Cu) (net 29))
 (segment (start 118.910998 101.6) (end 130.81 101.6) (width 0.25) (layer B.Cu) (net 29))
 (segment (start 116.84 59.69) (end 116.84 99.529002) (width 0.25) (layer B.Cu) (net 29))
 (segment (start 116.84 99.529002) (end 118.910998 101.6) (width 0.25) (layer B.Cu) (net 29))
 (segment (start 131.895009 87.583639) (end 129.40137 85.09) (width 0.25) (layer F.Cu) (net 29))
 (segment (start 129.40137 85.09) (end 128.27 85.09) (width 0.25) (layer F.Cu) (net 29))
 (segment (start 131.895009 100.514991) (end 131.895009 87.583639) (width 0.25) (layer F.Cu) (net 29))
 (segment (start 130.81 101.6) (end 131.895009 100.514991) (width 0.25) (layer F.Cu) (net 29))
 (segment (start 116.389991 101.618993) (end 116.389991 57.600009) (width 0.25) (layer B.Cu) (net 30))
 (segment (start 116.389991 57.600009) (end 119.38 54.61) (width 0.25) (layer B.Cu) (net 30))
 (segment (start 118.815999 104.045001) (end 116.389991 101.618993) (width 0.25) (layer B.Cu) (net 30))
 (segment (start 134.523591 104.045001) (end 118.815999 104.045001) (width 0.25) (layer B.Cu) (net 30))
 (segment (start 138.42859 107.95) (end 134.523591 104.045001) (width 0.25) (layer B.Cu) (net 30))
 (segment (start 143.51 107.95) (end 138.42859 107.95) (width 0.25) (layer B.Cu) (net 30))
 (segment (start 128.27 91.835002) (end 128.27 92.71) (width 0.25) (layer F.Cu) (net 23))
 (segment (start 133.985 92.71) (end 128.27 92.71) (width 0.25) (layer B.Cu) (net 23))
 (segment (start 143.114998 101.6) (end 134.224998 92.71) (width 0.25) (layer B.Cu) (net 23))
 (segment (start 134.224998 92.71) (end 133.985 92.71) (width 0.25) (layer B.Cu) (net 23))
 (segment (start 146.05 101.6) (end 143.114998 101.6) (width 0.25) (layer B.Cu) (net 23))
 (segment (start 147.410001 50.509999) (end 147.410001 100.239999) (width 0.25) (layer B.Cu) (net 23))
 (segment (start 147.410001 100.239999) (end 146.05 101.6) (width 0.25) (layer B.Cu) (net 23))
 (segment (start 119.38 52.07) (end 123.19 48.26) (width 0.25) (layer B.Cu) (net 23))
 (segment (start 145.160002 48.26) (end 147.410001 50.509999) (width 0.25) (layer B.Cu) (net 23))
 (segment (start 123.19 48.26) (end 145.160002 48.26) (width 0.25) (layer B.Cu) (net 23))
 (segment (start 123.19 49.53) (end 136.525 62.865) (width 0.25) (layer F.Cu) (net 20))
 (segment (start 119.38 49.53) (end 123.19 49.53) (width 0.25) (layer F.Cu) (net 20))
 (segment (start 139.065 62.865) (end 141.605 62.865) (width 0.25) (layer F.Cu) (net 20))
 (segment (start 141.605 62.865) (end 144.145 62.865) (width 0.25) (layer F.Cu) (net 20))
 (segment (start 143.51 95.25) (end 139.7 91.44) (width 0.25) (layer B.Cu) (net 20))
 (segment (start 139.7 91.44) (end 139.7 77.47) (width 0.25) (layer B.Cu) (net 20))
 (via (at 139.7 77.47) (size 0.8) (drill 0.4) (layers F.Cu B.Cu) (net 20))
 (segment (start 137.704999 62.955001) (end 137.795 62.865) (width 0.25) (layer F.Cu) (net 20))
 (segment (start 136.525 62.865) (end 137.795 62.865) (width 0.25) (layer F.Cu) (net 20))
 (segment (start 137.704999 75.474999) (end 137.704999 62.955001) (width 0.25) (layer F.Cu) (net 20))
 (segment (start 139.7 77.47) (end 137.704999 75.474999) (width 0.25) (layer F.Cu) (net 20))
 (segment (start 137.795 62.865) (end 139.065 62.865) (width 0.25) (layer F.Cu) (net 20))
 (segment (start 133.985 71.755) (end 133.985 49.53) (width 0.25) (layer B.Cu) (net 35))
 (segment (start 128.27 77.47) (end 133.985 71.755) (width 0.25) (layer B.Cu) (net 35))
 (segment (start 140.579999 53.584999) (end 136.525 49.53) (width 0.25) (layer B.Cu) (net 31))
 (segment (start 140.579999 66.430001) (end 140.579999 53.584999) (width 0.25) (layer B.Cu) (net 31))
 (segment (start 139.065 67.945) (end 140.579999 66.430001) (width 0.25) (layer B.Cu) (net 31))
 (segment (start 139.065 67.945) (end 132.715 74.295) (width 0.25) (layer B.Cu) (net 31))
 (via (at 132.715 74.295) (size 0.8) (drill 0.4) (layers F.Cu B.Cu) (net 31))
 (segment (start 132.715 74.295) (end 132.715 80.01) (width 0.25) (layer F.Cu) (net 31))
 (segment (start 132.715 80.01) (end 132.715 82.55) (width 0.25) (layer F.Cu) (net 31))
 (via (at 132.715 82.55) (size 0.8) (drill 0.4) (layers F.Cu B.Cu) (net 31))
 (segment (start 132.715 82.55) (end 128.27 82.55) (width 0.25) (layer B.Cu) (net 31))
 (segment (start 143.51 77.47) (end 146.685 74.295) (width 0.25) (layer B.Cu) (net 6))
 (via (at 146.685 55.245) (size 0.8) (drill 0.4) (layers F.Cu B.Cu) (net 6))
 (segment (start 146.685 74.295) (end 146.685 55.245) (width 0.25) (layer B.Cu) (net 6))
 (segment (start 146.685 55.245) (end 146.685 53.975) (width 0.25) (layer F.Cu) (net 6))
 (segment (start 146.685 53.975) (end 145.415 52.705) (width 0.25) (layer F.Cu) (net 6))
 (segment (start 142.24 52.705) (end 139.065 49.53) (width 0.25) (layer F.Cu) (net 6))
 (segment (start 145.415 52.705) (end 142.24 52.705) (width 0.25) (layer F.Cu) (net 6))
 (segment (start 142.630001 50.555001) (end 141.605 49.53) (width 0.25) (layer B.Cu) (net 33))
 (segment (start 142.630001 66.919999) (end 142.630001 50.555001) (width 0.25) (layer B.Cu) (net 33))
 (segment (start 141.605 67.945) (end 142.630001 66.919999) (width 0.25) (layer B.Cu) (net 33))
 (segment (start 128.27 80.01) (end 130.175 78.105) (width 0.25) (layer F.Cu) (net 33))
 (via (at 130.175 77.47) (size 0.8) (drill 0.4) (layers F.Cu B.Cu) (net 33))
 (segment (start 130.175 78.105) (end 130.175 77.47) (width 0.25) (layer F.Cu) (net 33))
 (segment (start 130.175 77.47) (end 132.08 75.565) (width 0.25) (layer B.Cu) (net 33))
 (segment (start 133.985 75.565) (end 141.605 67.945) (width 0.25) (layer B.Cu) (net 33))
 (segment (start 132.08 75.565) (end 133.985 75.565) (width 0.25) (layer B.Cu) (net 33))
 (segment (start 145.170001 66.919999) (end 145.170001 50.555001) (width 0.25) (layer B.Cu) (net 8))
 (segment (start 145.170001 50.555001) (end 144.145 49.53) (width 0.25) (layer B.Cu) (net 8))
 (segment (start 144.145 67.945) (end 145.170001 66.919999) (width 0.25) (layer B.Cu) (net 8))
 (segment (start 144.844999 78.675001) (end 143.51 80.01) (width 0.25) (layer F.Cu) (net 8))
 (segment (start 144.844999 68.644999) (end 144.844999 78.675001) (width 0.25) (layer F.Cu) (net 8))
 (segment (start 144.145 67.945) (end 144.844999 68.644999) (width 0.25) (layer F.Cu) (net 8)))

